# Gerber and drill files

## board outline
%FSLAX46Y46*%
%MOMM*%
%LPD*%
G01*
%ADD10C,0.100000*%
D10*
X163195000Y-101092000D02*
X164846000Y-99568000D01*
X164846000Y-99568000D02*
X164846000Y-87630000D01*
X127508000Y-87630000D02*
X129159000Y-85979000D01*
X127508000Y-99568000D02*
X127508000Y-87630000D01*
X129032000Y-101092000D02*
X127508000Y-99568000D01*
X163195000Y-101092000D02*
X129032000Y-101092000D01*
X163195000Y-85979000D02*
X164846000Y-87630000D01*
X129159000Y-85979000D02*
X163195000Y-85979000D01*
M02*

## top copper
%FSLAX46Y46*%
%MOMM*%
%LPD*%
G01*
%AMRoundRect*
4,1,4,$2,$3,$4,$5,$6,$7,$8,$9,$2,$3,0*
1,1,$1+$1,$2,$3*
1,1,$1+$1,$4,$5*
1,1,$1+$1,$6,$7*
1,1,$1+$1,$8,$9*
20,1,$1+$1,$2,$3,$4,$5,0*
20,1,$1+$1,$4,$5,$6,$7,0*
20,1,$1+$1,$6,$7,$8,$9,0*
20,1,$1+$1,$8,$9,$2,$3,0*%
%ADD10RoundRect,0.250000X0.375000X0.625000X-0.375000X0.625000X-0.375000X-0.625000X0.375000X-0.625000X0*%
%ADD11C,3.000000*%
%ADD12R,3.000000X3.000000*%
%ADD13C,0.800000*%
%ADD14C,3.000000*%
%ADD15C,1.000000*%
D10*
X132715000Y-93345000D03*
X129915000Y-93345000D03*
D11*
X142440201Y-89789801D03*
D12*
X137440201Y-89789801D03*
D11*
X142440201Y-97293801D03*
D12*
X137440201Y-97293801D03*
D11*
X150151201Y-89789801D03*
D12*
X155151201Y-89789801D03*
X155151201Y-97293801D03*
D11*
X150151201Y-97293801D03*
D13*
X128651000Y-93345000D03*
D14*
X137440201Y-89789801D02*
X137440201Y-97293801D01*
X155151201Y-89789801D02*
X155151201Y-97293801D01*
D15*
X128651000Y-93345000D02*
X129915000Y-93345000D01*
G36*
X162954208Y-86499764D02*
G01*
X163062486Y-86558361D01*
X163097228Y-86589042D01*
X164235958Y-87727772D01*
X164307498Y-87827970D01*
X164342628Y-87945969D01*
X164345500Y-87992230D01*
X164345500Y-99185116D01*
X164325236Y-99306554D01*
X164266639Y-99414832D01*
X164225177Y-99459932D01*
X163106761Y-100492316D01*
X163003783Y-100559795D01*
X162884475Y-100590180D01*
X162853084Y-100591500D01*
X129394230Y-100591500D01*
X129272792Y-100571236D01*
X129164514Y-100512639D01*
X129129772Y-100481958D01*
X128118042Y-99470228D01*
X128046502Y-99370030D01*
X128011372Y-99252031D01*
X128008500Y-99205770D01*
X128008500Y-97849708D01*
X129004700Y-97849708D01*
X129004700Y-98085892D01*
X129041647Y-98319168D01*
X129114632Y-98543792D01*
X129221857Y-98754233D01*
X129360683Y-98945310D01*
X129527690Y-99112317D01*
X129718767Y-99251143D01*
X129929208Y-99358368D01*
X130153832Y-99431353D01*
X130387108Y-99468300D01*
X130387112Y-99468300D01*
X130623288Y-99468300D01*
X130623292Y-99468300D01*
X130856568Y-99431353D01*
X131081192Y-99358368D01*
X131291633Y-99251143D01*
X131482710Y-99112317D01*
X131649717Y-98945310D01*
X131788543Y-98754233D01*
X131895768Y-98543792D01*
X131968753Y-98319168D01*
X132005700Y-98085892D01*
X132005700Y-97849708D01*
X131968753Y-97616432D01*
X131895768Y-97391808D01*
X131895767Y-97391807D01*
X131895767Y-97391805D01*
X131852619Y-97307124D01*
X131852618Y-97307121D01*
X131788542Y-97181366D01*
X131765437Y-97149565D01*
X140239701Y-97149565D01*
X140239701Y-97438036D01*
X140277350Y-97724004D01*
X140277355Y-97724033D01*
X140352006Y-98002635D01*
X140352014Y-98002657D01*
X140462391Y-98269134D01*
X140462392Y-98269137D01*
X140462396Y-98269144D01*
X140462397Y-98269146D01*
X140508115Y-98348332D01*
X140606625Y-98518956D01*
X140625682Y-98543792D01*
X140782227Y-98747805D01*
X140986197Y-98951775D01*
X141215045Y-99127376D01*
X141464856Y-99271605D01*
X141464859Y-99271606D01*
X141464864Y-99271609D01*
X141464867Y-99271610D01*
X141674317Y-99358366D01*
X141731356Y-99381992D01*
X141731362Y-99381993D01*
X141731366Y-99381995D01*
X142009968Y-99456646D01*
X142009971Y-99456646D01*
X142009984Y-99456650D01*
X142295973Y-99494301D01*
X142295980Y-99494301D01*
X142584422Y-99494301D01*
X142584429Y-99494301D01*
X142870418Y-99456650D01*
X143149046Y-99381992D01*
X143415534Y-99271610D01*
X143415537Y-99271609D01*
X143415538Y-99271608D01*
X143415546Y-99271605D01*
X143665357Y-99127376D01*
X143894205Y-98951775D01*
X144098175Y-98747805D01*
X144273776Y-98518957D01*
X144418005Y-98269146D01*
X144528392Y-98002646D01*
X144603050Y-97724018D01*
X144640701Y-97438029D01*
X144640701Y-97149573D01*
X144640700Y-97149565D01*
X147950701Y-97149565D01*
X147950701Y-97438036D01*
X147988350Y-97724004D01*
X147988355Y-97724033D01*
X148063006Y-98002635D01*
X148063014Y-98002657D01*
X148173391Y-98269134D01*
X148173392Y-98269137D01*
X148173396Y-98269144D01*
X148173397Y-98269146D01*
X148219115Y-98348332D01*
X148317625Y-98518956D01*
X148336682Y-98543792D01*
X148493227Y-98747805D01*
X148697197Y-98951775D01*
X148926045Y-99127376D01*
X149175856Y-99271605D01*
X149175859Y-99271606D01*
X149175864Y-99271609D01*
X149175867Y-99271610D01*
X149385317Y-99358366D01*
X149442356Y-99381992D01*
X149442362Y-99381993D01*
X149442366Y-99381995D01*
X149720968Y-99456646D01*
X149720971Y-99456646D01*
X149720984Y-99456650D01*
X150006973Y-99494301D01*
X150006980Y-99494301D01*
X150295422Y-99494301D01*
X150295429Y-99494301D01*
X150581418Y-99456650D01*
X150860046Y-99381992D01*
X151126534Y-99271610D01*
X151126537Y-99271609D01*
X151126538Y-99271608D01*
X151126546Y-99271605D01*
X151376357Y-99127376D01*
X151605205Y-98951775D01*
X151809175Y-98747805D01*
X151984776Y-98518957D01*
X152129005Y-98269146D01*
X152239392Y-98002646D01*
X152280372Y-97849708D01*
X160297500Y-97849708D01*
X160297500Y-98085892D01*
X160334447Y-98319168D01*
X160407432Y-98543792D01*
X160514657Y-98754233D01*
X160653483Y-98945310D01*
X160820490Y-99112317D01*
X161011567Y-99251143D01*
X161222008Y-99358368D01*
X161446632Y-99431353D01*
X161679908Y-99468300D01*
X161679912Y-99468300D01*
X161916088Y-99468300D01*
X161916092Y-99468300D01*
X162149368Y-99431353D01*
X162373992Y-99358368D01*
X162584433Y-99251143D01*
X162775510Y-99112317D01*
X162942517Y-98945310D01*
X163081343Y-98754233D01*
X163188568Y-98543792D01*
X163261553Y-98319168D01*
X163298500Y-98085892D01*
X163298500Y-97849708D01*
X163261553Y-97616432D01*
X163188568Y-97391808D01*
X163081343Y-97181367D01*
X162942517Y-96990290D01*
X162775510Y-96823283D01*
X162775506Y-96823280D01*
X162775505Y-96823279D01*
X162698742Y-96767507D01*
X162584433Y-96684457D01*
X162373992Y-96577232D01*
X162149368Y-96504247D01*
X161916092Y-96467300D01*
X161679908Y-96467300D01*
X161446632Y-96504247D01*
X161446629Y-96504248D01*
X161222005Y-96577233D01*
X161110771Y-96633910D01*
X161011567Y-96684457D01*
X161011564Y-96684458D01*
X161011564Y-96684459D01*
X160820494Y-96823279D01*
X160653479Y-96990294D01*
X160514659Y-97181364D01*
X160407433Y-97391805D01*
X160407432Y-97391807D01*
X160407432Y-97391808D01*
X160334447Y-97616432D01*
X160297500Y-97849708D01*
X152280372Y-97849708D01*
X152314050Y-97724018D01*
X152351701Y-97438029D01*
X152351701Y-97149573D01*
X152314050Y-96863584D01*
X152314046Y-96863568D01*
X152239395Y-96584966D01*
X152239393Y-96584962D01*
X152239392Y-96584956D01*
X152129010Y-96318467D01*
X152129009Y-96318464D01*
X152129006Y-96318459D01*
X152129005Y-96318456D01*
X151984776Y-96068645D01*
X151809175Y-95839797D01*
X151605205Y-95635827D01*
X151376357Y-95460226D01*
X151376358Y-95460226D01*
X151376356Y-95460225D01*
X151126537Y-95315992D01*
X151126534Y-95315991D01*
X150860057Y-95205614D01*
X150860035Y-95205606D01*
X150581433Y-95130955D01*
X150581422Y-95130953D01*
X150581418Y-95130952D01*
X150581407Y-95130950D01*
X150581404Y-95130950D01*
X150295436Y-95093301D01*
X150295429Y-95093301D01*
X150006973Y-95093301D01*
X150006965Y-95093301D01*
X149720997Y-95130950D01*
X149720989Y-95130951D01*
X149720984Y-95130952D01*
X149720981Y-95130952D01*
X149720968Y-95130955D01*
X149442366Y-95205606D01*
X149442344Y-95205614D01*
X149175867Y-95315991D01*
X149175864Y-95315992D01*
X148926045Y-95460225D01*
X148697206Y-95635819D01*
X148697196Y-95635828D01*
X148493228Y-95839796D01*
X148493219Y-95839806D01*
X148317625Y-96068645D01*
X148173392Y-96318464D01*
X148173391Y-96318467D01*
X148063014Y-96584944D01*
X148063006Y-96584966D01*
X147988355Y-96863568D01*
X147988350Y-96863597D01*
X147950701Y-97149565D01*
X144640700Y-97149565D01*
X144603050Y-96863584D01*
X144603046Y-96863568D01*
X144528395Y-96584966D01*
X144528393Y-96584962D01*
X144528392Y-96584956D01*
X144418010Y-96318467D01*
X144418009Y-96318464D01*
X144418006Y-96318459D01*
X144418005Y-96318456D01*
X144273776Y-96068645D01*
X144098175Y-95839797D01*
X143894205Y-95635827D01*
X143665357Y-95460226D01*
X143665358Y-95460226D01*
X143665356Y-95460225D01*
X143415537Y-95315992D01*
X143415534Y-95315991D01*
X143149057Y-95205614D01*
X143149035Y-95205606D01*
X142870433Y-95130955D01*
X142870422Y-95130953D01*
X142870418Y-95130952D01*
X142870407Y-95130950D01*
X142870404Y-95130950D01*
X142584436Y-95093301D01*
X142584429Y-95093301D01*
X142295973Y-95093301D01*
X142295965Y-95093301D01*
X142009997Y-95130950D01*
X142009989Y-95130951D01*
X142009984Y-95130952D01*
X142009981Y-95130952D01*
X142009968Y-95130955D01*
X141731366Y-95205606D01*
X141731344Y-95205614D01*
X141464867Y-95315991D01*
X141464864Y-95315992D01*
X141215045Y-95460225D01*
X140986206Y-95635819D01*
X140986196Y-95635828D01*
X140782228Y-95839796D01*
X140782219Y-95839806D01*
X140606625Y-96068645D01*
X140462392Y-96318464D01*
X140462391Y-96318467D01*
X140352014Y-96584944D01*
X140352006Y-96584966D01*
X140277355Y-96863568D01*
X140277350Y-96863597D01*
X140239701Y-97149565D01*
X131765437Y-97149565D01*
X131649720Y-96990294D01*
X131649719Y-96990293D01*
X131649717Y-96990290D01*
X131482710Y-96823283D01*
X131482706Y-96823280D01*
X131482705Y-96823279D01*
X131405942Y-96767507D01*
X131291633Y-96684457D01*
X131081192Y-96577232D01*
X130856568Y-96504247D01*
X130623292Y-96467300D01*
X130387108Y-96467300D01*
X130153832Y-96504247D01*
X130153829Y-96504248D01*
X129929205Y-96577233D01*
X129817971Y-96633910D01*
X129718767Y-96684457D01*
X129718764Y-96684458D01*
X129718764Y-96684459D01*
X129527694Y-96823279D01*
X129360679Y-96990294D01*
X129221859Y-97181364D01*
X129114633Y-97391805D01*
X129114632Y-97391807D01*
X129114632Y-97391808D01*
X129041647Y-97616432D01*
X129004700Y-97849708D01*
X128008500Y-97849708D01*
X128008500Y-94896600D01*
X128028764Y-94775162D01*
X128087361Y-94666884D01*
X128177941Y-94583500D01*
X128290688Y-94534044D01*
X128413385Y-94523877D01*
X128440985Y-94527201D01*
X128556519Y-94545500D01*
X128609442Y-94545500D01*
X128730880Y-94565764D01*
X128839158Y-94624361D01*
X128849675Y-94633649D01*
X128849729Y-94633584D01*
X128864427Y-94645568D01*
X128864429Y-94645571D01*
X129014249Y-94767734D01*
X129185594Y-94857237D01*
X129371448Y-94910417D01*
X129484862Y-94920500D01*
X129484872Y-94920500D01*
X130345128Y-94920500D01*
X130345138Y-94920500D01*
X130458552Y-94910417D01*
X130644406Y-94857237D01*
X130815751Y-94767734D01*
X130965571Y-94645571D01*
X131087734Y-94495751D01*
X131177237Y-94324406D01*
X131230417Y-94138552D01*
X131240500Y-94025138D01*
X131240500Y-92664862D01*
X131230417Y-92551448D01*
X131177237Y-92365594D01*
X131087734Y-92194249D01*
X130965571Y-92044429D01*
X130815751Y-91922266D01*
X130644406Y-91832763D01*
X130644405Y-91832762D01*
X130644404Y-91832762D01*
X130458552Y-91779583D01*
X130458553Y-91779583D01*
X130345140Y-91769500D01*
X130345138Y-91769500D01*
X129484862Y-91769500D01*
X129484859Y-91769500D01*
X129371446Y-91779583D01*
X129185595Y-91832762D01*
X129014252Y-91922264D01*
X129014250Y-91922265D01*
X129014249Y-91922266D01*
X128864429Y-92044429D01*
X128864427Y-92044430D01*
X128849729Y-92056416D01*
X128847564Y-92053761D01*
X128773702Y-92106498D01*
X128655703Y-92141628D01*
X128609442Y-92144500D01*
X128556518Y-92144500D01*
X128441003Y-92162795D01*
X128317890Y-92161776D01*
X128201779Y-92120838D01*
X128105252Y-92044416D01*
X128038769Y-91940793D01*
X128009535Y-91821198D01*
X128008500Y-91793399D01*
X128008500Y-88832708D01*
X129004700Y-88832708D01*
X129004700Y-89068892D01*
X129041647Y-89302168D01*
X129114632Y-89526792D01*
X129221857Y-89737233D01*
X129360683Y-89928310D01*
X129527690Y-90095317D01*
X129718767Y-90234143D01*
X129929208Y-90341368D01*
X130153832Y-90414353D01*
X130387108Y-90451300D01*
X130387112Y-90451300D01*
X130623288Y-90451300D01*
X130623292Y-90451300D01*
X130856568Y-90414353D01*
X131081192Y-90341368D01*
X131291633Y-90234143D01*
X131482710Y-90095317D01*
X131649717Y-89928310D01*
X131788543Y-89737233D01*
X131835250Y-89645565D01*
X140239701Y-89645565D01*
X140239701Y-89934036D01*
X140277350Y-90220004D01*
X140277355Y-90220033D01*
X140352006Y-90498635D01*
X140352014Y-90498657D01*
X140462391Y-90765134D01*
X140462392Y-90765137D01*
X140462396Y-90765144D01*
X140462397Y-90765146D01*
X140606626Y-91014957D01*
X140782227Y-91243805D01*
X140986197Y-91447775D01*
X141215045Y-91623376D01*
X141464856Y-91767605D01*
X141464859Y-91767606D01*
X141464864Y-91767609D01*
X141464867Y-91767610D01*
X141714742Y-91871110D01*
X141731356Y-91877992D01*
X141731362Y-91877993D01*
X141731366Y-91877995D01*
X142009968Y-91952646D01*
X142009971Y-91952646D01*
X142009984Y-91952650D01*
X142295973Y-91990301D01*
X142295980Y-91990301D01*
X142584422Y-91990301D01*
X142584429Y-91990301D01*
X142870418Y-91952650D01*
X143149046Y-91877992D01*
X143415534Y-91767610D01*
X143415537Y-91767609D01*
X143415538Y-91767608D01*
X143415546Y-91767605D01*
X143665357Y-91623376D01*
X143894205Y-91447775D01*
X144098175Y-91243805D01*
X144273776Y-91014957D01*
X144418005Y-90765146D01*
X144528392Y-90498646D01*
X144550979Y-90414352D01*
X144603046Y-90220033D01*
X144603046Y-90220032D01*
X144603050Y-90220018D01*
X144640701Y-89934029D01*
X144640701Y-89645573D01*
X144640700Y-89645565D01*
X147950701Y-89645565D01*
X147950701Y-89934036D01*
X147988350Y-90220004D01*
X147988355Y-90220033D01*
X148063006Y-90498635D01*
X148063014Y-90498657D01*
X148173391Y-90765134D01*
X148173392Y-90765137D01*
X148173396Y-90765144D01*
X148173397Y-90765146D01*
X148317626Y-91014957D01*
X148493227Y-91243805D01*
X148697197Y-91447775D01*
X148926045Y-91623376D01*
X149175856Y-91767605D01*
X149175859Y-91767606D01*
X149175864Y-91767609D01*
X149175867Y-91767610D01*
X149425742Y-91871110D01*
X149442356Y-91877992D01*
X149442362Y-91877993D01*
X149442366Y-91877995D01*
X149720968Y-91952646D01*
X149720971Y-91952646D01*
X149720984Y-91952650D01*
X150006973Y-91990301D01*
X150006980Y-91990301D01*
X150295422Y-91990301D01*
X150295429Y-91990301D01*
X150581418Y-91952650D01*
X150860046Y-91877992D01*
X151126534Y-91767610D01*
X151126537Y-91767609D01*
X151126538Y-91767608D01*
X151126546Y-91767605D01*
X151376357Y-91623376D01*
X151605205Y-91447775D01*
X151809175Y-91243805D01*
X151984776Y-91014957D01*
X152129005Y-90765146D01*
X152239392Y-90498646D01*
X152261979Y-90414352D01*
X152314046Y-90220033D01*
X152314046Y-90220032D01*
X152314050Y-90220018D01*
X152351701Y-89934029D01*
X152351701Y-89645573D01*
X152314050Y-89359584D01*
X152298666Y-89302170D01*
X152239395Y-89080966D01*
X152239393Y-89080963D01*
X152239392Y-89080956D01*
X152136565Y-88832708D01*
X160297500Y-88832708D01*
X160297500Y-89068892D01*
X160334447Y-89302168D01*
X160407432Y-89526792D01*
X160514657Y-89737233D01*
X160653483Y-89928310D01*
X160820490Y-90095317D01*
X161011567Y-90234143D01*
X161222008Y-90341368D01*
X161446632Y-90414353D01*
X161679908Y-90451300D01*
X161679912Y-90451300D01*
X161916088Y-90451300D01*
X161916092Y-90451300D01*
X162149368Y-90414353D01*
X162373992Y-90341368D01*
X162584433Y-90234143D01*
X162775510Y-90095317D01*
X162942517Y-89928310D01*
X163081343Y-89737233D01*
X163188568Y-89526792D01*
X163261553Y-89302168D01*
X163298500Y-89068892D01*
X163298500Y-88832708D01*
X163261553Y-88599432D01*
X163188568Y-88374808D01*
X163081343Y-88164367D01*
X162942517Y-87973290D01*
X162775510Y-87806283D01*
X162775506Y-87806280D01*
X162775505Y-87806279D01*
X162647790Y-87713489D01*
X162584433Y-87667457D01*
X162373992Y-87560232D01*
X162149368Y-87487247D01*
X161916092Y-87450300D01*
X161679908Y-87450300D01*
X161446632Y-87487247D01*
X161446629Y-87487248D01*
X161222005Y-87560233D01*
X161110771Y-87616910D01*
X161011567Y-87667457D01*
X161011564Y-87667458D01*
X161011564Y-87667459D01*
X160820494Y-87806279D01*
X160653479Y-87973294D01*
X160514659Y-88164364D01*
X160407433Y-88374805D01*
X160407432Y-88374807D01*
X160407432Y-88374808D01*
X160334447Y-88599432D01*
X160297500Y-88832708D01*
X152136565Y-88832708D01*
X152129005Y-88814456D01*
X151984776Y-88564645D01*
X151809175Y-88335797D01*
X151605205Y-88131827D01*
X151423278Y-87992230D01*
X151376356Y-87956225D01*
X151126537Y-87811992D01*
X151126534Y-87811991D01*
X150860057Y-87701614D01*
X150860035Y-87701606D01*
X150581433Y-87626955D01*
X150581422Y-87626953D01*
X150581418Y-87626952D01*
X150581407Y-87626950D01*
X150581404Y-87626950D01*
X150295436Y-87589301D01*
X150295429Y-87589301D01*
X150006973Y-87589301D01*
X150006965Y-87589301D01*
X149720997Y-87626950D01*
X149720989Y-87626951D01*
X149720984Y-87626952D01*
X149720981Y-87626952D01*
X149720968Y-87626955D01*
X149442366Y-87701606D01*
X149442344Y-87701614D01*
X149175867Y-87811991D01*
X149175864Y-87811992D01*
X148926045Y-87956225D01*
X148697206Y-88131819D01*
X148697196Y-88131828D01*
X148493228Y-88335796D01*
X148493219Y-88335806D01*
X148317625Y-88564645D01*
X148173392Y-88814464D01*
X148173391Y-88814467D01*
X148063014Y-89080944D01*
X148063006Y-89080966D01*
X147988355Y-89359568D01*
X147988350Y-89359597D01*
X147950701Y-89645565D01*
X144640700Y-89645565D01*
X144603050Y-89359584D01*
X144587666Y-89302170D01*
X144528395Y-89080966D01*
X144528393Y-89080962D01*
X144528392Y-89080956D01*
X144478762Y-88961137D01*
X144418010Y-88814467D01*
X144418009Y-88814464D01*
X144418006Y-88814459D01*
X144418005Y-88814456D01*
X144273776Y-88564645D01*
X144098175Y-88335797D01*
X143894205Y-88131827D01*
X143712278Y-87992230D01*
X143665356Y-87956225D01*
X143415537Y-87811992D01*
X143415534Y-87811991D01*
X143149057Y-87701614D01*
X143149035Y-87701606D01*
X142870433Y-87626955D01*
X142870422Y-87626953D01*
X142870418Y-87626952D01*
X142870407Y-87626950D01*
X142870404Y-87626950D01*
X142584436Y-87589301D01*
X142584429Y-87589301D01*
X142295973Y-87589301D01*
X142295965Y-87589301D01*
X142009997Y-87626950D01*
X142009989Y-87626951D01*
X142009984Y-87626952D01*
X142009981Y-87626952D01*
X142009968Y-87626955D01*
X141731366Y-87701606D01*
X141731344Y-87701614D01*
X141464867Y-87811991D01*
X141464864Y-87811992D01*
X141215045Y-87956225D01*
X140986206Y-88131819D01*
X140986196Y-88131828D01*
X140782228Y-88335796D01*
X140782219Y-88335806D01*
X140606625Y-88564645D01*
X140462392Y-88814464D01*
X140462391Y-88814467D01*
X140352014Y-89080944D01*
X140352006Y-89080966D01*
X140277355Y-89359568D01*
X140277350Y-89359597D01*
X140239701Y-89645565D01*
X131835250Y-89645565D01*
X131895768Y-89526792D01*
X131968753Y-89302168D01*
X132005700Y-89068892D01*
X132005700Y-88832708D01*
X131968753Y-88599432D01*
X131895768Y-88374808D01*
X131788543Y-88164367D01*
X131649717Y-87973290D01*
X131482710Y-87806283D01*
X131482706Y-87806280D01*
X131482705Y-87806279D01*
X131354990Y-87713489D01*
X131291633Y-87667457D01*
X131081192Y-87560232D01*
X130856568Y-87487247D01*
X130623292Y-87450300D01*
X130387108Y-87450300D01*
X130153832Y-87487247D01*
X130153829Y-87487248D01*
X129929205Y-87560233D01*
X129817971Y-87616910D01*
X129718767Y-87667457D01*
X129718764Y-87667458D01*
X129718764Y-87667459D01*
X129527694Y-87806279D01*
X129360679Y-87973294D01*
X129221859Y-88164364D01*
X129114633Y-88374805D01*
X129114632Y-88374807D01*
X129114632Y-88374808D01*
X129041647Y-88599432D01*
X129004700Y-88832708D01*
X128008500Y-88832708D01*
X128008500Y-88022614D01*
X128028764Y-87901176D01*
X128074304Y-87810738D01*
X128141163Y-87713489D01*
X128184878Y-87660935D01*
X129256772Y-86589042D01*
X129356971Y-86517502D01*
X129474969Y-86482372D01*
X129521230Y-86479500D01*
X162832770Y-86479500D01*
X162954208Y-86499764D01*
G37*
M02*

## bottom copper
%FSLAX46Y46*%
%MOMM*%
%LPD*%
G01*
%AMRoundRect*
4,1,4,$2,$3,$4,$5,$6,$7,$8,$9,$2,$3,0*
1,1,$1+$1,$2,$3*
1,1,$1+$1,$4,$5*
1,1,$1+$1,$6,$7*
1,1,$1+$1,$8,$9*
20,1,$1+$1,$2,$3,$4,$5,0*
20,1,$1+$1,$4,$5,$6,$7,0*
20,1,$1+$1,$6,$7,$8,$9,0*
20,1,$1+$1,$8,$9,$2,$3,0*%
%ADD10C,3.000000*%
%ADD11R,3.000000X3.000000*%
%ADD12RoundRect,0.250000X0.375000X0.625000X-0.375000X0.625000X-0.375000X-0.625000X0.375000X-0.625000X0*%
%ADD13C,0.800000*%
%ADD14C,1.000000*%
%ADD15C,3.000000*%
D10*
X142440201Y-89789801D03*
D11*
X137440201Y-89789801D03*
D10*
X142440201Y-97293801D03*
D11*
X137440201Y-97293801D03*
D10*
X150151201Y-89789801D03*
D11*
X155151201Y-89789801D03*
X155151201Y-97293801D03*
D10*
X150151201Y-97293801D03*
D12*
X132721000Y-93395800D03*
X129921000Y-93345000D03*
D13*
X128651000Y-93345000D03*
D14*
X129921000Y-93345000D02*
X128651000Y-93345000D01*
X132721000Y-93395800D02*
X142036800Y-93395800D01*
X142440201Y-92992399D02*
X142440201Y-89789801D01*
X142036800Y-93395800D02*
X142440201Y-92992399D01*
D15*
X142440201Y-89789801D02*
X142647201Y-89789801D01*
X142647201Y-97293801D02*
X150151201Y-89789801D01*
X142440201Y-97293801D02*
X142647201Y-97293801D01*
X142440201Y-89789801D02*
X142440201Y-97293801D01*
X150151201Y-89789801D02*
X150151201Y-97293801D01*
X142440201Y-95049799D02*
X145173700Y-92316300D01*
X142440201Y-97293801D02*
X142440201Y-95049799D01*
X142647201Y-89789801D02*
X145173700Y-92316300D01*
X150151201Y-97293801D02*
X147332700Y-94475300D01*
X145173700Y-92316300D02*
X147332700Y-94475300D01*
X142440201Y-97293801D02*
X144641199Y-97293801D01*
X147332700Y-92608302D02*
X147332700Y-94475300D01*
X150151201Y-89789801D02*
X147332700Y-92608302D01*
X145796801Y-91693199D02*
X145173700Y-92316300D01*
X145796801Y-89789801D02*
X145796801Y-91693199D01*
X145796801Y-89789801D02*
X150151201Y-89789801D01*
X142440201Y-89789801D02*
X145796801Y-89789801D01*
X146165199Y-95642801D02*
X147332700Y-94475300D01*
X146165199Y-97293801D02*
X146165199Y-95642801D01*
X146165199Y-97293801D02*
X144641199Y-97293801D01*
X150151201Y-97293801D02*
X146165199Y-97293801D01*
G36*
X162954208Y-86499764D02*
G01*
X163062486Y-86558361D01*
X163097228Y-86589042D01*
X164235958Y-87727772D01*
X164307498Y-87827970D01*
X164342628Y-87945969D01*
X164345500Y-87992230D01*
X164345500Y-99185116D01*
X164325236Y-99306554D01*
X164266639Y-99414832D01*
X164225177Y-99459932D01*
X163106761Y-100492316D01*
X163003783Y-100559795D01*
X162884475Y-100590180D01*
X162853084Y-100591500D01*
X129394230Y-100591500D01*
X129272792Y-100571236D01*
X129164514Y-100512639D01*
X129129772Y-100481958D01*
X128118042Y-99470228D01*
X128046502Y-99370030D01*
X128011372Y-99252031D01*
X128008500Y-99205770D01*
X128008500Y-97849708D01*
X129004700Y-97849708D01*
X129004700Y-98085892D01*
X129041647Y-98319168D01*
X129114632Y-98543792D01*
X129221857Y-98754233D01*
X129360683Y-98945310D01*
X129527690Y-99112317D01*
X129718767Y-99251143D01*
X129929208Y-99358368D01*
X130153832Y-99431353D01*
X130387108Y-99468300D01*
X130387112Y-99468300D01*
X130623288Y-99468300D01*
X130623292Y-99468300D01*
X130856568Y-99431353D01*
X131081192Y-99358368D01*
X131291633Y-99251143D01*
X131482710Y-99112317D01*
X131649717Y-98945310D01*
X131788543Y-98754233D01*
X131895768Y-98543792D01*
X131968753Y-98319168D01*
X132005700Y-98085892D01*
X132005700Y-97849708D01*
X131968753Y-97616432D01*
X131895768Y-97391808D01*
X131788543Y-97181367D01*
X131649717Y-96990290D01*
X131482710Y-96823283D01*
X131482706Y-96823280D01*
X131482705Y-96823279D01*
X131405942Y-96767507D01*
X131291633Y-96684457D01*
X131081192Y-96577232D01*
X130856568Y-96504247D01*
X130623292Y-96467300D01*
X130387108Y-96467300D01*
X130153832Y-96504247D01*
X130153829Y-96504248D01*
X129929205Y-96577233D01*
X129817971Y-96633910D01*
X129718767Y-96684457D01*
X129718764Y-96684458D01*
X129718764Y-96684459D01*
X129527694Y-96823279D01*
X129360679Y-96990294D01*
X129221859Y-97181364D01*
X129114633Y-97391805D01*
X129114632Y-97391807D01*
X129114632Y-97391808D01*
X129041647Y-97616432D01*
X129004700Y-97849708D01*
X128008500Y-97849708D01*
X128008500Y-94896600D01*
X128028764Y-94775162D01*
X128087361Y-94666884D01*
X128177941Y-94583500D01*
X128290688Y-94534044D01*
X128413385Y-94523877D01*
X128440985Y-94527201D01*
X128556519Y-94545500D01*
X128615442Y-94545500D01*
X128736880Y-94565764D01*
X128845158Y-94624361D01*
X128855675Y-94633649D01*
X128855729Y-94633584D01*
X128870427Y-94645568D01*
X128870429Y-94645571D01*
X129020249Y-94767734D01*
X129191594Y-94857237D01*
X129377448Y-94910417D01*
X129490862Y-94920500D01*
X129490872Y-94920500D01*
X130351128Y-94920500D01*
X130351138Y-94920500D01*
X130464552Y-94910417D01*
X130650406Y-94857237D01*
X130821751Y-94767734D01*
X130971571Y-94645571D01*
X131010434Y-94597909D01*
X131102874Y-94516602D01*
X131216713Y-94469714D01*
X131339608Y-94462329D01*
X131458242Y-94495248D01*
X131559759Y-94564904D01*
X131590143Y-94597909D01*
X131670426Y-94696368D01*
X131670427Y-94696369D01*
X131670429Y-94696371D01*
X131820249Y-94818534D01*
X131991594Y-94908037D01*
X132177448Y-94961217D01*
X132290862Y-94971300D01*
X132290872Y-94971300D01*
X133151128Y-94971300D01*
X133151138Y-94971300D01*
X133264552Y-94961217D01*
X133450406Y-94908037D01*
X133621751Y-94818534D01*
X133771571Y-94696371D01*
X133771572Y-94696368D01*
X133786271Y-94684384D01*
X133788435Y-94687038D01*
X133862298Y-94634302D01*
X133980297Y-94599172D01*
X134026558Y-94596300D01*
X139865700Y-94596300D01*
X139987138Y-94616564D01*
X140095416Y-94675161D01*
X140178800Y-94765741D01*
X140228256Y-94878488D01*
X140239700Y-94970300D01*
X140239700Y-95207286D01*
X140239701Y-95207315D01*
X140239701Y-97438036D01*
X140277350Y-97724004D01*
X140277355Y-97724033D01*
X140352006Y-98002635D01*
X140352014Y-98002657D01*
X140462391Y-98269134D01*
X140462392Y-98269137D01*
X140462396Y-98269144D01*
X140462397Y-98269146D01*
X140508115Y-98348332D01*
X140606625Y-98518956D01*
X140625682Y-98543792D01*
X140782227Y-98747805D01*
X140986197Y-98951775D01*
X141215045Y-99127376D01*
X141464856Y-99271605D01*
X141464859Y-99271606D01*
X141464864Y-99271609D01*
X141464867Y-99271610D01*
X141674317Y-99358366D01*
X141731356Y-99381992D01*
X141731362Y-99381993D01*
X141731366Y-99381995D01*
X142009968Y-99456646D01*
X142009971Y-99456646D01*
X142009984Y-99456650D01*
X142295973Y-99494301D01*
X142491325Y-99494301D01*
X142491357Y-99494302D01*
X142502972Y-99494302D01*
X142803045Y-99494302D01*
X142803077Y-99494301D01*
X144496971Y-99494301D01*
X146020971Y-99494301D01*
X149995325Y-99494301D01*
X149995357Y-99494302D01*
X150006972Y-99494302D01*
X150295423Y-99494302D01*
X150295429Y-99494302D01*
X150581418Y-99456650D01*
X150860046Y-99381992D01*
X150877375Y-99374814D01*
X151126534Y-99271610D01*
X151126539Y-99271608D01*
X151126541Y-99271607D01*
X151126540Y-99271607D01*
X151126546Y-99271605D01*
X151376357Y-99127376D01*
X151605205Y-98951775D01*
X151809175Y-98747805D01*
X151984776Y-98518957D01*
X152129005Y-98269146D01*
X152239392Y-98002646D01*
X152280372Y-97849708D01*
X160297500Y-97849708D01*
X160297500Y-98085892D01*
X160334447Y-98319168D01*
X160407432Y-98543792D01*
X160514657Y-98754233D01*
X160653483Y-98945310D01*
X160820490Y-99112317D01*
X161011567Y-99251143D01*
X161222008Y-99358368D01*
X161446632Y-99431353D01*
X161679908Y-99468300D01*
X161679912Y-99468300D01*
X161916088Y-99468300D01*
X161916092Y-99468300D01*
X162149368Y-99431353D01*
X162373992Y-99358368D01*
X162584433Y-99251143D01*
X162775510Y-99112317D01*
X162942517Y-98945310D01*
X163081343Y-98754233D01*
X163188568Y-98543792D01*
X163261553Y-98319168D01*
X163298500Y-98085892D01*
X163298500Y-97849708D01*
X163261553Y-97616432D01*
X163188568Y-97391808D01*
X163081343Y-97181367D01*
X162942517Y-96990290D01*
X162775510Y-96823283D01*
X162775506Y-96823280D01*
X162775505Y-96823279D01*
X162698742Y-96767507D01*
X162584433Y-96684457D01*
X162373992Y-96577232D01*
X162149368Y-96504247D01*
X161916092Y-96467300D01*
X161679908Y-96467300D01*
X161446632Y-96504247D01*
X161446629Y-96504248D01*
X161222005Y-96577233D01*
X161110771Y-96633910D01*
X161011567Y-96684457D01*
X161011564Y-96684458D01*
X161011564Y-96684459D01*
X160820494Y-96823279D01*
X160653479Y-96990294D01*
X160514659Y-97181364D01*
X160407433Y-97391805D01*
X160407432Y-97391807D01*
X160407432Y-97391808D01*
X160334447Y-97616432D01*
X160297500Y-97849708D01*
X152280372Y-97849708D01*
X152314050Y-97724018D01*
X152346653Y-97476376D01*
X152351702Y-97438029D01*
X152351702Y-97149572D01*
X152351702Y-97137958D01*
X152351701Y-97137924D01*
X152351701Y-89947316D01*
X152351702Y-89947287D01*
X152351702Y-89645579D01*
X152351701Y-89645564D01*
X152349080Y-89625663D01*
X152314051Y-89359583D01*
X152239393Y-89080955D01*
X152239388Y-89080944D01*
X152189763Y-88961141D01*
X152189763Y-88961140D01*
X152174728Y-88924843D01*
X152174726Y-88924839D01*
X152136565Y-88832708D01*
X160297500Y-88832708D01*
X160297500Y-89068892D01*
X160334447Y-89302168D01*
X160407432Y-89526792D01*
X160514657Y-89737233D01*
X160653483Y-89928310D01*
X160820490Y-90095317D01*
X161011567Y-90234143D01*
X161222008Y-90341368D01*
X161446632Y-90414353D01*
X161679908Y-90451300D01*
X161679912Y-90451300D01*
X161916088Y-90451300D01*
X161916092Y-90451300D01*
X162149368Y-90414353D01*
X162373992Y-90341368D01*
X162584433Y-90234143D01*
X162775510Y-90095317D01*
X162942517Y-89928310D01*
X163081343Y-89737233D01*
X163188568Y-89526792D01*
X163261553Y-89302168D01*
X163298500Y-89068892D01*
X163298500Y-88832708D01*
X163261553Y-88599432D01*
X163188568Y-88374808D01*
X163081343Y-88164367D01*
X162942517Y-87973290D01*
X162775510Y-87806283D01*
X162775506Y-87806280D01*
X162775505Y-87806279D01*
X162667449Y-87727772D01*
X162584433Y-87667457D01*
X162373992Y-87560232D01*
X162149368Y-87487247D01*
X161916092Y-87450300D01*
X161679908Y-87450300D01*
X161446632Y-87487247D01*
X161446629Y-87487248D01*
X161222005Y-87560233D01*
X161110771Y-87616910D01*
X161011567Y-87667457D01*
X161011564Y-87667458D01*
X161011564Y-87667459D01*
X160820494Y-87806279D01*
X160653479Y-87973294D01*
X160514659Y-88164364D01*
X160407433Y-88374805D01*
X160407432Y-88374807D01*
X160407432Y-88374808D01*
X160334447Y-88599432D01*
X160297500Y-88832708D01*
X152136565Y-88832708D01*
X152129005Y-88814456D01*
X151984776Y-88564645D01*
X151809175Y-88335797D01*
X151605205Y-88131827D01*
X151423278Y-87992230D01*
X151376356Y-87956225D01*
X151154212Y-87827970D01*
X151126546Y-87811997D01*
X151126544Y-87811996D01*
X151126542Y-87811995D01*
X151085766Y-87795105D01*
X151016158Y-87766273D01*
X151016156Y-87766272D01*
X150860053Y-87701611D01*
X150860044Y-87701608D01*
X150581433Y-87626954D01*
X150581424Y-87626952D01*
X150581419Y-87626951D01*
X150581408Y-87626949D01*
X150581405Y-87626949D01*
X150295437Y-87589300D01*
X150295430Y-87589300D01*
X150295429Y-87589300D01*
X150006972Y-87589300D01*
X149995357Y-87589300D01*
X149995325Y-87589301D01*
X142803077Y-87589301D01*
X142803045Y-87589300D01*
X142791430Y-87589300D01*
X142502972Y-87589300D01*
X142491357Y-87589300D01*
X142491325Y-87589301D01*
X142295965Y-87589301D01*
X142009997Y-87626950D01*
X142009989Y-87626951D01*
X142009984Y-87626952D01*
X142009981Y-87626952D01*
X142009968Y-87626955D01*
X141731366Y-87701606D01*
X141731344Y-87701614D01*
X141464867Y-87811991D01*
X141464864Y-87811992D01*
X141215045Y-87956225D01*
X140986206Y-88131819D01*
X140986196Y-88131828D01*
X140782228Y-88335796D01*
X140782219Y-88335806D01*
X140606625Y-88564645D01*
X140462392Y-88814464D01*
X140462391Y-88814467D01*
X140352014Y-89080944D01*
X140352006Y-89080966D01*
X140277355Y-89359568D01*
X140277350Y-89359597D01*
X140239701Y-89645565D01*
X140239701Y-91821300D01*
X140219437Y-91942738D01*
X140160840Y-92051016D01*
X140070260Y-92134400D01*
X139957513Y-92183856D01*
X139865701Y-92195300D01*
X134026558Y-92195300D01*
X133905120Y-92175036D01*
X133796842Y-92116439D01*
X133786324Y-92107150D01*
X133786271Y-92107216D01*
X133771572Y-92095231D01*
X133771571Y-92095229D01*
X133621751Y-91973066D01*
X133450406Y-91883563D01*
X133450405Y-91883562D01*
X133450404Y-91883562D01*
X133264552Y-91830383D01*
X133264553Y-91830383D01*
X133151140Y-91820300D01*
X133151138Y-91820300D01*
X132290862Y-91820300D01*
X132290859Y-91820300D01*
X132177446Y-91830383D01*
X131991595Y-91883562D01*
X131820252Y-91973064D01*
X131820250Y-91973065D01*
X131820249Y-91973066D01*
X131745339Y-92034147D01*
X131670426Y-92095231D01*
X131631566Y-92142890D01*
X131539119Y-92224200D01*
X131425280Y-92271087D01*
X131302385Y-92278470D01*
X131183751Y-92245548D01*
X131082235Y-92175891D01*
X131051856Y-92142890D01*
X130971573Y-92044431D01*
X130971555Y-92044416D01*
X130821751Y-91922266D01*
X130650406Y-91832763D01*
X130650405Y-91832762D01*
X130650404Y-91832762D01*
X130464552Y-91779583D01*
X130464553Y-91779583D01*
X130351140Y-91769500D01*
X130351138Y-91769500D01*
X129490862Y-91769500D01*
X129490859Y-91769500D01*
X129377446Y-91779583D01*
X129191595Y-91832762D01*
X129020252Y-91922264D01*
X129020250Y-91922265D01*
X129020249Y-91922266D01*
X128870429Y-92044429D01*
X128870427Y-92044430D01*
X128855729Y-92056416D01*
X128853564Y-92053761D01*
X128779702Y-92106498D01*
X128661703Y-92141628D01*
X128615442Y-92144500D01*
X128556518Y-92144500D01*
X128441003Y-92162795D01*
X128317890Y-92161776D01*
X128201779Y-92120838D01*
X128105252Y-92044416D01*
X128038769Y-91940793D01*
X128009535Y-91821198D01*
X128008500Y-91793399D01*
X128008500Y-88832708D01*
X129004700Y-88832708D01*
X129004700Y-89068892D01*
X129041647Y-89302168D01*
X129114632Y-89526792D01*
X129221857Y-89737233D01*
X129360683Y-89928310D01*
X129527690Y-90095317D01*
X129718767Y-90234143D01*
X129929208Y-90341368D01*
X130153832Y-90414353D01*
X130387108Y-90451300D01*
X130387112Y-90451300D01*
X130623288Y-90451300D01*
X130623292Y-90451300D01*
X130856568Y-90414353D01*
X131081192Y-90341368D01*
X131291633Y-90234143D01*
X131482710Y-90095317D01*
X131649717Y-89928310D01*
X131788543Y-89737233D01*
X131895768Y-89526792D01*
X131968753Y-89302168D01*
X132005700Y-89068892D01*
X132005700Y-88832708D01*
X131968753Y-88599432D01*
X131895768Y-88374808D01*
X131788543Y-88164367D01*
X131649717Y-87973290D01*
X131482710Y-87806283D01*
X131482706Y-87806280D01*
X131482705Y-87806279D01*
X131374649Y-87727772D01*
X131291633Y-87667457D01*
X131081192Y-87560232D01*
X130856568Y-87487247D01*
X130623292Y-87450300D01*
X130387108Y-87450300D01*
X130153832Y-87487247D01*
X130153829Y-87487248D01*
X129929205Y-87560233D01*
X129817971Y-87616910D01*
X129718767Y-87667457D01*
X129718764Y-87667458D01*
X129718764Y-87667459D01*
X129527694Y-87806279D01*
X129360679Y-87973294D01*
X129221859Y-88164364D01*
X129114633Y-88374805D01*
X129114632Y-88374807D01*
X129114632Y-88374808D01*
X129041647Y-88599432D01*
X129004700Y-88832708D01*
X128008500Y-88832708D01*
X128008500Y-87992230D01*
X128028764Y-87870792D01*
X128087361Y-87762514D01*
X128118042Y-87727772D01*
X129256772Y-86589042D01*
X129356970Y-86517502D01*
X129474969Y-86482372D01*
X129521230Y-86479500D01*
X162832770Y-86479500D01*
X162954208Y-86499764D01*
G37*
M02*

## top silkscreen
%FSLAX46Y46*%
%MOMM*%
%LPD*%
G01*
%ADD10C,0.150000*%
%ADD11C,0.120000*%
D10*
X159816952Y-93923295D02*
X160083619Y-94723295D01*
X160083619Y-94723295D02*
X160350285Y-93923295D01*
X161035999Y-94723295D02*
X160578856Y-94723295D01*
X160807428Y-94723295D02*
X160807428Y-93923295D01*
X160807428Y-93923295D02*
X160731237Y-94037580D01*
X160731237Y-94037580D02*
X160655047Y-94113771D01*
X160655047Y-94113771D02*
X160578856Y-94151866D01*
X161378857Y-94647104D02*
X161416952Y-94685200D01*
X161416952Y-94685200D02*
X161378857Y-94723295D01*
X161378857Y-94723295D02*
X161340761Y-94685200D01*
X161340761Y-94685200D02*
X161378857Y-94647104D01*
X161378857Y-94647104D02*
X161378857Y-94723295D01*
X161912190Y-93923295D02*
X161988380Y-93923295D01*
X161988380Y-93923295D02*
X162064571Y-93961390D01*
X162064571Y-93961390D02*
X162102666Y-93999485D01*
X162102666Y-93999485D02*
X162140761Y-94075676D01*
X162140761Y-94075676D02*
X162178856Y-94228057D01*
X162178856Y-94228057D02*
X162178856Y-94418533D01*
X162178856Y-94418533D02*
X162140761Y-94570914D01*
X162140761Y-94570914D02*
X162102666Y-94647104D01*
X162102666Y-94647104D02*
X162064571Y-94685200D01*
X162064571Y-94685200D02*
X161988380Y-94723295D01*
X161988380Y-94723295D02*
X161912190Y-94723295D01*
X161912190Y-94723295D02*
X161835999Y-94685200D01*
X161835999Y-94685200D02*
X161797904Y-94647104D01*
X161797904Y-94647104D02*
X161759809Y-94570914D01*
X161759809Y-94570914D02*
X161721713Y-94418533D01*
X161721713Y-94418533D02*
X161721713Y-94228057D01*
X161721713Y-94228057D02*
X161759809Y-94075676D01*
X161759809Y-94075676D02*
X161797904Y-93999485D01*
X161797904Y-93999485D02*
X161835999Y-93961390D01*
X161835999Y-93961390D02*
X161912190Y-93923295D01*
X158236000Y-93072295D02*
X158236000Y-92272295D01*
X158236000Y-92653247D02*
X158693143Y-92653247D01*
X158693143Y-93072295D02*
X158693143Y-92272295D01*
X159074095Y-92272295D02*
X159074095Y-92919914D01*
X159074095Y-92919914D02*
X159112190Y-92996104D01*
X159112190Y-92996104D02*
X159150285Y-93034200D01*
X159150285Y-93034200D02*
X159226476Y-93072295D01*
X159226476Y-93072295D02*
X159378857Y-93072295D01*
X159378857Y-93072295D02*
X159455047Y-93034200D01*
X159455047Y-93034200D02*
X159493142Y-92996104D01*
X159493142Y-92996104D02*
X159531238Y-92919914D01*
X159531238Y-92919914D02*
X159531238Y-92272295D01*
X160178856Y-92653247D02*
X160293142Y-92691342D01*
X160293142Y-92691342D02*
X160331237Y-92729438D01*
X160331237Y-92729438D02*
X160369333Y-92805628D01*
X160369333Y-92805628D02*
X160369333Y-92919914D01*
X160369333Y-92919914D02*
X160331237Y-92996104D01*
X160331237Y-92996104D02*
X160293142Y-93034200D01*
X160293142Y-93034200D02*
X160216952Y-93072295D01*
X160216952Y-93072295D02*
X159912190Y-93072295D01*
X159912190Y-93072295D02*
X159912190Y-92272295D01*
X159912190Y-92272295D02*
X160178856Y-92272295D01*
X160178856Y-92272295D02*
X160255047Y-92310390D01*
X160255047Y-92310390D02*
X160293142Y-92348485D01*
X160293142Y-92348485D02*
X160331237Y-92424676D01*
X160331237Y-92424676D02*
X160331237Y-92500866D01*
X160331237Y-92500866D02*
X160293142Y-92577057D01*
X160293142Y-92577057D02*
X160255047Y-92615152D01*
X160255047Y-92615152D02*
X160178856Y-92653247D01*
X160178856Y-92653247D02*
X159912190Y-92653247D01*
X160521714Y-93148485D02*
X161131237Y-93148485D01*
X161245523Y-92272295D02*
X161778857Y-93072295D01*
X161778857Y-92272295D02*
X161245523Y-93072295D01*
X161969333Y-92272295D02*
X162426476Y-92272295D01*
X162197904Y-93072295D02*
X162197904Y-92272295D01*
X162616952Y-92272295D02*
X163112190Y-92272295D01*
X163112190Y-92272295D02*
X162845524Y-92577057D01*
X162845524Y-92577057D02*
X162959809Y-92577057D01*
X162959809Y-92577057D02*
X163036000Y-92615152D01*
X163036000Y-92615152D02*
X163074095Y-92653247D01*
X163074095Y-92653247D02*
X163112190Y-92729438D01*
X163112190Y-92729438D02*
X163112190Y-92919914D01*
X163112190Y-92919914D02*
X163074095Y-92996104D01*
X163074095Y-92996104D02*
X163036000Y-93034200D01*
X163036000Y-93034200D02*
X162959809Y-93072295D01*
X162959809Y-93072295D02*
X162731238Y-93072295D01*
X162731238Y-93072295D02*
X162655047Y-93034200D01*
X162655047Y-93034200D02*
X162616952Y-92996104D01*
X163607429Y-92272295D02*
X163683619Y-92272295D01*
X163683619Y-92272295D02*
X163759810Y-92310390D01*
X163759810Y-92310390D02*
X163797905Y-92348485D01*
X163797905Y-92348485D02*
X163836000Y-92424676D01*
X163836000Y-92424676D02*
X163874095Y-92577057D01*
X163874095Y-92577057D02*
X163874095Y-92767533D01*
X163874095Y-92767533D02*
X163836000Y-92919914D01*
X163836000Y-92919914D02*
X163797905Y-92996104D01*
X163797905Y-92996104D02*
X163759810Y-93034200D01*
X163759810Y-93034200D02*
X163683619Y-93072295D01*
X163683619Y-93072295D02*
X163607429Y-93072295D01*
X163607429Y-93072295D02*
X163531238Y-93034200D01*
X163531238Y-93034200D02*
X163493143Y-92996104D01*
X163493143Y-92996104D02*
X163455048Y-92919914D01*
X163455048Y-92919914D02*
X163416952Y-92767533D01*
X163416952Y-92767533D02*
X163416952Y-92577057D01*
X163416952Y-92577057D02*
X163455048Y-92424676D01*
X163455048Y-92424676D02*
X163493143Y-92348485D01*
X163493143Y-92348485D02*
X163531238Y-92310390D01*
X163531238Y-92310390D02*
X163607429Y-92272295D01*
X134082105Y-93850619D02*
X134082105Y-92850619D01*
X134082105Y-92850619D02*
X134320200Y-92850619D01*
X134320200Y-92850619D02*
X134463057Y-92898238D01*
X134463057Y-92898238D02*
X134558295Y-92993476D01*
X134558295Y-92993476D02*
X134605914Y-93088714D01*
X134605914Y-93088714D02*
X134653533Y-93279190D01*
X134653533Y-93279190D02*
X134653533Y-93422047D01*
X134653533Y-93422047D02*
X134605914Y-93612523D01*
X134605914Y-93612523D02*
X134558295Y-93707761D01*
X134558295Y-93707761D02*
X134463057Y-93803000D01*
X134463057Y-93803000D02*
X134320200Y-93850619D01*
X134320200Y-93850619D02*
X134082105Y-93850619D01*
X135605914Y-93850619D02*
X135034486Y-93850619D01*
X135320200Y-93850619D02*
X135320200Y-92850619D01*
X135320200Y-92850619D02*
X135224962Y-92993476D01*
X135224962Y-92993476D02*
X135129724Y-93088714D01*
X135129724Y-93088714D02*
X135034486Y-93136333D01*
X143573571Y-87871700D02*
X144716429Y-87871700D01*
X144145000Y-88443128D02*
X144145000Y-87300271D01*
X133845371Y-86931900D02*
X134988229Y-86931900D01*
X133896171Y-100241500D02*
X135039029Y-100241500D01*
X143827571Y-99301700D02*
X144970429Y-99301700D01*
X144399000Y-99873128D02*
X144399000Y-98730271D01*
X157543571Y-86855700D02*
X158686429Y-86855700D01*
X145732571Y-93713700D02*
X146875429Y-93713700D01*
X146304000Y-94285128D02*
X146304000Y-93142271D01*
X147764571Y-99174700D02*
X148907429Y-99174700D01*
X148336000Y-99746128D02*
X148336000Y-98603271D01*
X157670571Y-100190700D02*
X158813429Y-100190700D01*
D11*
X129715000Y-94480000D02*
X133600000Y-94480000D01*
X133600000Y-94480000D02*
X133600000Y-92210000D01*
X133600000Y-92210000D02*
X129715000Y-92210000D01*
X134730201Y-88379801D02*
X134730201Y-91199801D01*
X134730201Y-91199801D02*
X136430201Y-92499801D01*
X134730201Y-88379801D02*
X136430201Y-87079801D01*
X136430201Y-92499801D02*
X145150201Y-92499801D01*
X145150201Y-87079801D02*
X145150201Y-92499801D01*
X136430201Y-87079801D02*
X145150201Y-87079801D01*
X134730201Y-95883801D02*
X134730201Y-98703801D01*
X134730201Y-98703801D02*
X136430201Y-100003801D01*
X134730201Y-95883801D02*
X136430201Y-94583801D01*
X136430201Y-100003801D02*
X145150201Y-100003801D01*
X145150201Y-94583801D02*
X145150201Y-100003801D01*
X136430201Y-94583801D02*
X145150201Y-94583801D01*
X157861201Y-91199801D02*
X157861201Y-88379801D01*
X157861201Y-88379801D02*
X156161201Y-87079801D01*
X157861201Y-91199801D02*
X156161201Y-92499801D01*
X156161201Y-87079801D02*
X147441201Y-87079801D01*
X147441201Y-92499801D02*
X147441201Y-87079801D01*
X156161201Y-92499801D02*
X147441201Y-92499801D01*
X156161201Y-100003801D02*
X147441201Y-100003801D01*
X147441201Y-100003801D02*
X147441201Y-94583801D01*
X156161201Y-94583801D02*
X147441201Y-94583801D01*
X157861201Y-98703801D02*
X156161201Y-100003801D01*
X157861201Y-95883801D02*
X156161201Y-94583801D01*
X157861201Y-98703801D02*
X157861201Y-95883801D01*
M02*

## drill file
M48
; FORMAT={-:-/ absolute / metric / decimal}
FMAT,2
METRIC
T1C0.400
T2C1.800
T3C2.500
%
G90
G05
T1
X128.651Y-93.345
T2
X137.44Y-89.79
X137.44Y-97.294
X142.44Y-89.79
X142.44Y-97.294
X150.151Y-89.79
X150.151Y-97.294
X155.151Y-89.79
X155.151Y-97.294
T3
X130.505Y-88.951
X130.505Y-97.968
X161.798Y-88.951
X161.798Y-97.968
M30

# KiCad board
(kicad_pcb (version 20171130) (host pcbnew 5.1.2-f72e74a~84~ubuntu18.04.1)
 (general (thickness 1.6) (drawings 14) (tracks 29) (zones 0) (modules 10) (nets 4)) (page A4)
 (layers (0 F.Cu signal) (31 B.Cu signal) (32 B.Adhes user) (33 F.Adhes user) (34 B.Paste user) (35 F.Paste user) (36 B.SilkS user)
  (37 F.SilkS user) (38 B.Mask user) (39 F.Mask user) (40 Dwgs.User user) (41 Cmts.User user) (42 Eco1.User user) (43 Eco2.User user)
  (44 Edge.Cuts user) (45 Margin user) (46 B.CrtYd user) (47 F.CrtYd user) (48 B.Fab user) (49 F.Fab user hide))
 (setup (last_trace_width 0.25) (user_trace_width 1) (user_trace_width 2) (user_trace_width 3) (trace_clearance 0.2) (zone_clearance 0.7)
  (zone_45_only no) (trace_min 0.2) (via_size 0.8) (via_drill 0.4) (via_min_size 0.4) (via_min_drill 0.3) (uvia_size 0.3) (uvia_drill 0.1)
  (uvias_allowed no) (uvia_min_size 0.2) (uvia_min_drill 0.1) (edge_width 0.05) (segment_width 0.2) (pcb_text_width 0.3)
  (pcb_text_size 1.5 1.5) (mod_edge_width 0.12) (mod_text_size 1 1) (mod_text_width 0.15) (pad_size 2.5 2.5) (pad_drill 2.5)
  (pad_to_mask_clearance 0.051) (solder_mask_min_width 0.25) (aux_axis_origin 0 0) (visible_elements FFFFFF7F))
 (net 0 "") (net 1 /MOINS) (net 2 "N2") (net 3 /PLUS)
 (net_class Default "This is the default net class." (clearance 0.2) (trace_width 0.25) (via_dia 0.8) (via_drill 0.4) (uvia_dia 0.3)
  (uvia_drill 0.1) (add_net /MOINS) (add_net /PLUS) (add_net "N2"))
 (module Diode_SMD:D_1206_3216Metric (layer F.Cu) (at 131.315 93.345 180)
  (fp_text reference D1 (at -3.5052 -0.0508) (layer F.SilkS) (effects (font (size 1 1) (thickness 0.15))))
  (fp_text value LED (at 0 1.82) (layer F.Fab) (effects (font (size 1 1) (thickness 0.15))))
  (fp_line (start 1.6 -1.135) (end -2.285 -1.135) (layer F.SilkS) (width 0.12))
  (fp_line (start -2.285 -1.135) (end -2.285 1.135) (layer F.SilkS) (width 0.12))
  (fp_line (start -2.285 1.135) (end 1.6 1.135) (layer F.SilkS) (width 0.12))
  (pad 1 smd roundrect (at -1.4 0 180) (size 1.25 1.75) (layers F.Cu F.Paste F.Mask) (roundrect_rratio 0.2) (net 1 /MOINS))
  (pad 2 smd roundrect (at 1.4 0 180) (size 1.25 1.75) (layers F.Cu F.Paste F.Mask) (roundrect_rratio 0.2) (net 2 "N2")))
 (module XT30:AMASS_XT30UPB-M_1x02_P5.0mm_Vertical (layer F.Cu) (at 137.440201 89.789801)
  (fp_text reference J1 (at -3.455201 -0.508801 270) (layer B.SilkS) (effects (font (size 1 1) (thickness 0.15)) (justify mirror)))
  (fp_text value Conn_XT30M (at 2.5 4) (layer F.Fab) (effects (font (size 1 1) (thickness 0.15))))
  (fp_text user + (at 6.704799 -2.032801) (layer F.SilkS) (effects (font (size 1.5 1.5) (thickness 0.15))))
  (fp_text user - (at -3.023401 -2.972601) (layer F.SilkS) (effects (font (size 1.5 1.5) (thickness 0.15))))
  (fp_line (start -2.71 -1.41) (end -2.71 1.41) (layer F.SilkS) (width 0.12))
  (fp_line (start -2.71 1.41) (end -1.01 2.71) (layer F.SilkS) (width 0.12))
  (fp_line (start -2.71 -1.41) (end -1.01 -2.71) (layer F.SilkS) (width 0.12))
  (fp_line (start -1.01 2.71) (end 7.71 2.71) (layer F.SilkS) (width 0.12))
  (fp_line (start 7.71 -2.71) (end 7.71 2.71) (layer F.SilkS) (width 0.12))
  (fp_line (start -1.01 -2.71) (end 7.71 -2.71) (layer F.SilkS) (width 0.12))
  (pad 2 thru_hole circle (at 5 0) (size 3 3) (drill 1.8) (layers *.Cu *.Mask) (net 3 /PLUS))
  (pad 1 thru_hole rect (at 0 0) (size 3 3) (drill 1.8) (layers *.Cu *.Mask) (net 1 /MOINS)))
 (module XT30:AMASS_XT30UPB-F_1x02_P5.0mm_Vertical (layer F.Cu) (at 137.440201 97.293801)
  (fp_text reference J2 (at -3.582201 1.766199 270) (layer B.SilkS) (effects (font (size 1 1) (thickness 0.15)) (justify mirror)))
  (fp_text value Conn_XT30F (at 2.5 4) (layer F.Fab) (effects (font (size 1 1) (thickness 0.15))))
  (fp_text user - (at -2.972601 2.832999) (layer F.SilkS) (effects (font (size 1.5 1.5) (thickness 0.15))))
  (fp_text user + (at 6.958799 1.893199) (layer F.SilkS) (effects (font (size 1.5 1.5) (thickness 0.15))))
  (fp_line (start -2.71 -1.41) (end -2.71 1.41) (layer F.SilkS) (width 0.12))
  (fp_line (start -2.71 1.41) (end -1.01 2.71) (layer F.SilkS) (width 0.12))
  (fp_line (start -2.71 -1.41) (end -1.01 -2.71) (layer F.SilkS) (width 0.12))
  (fp_line (start -1.01 2.71) (end 7.71 2.71) (layer F.SilkS) (width 0.12))
  (fp_line (start 7.71 -2.71) (end 7.71 2.71) (layer F.SilkS) (width 0.12))
  (fp_line (start -1.01 -2.71) (end 7.71 -2.71) (layer F.SilkS) (width 0.12))
  (pad 2 thru_hole circle (at 5 0) (size 3 3) (drill 1.8) (layers *.Cu *.Mask) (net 3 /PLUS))
  (pad 1 thru_hole rect (at 0 0) (size 3 3) (drill 1.8) (layers *.Cu *.Mask) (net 1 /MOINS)))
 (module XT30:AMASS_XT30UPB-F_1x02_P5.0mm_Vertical (layer F.Cu) (at 155.151201 89.789801 180)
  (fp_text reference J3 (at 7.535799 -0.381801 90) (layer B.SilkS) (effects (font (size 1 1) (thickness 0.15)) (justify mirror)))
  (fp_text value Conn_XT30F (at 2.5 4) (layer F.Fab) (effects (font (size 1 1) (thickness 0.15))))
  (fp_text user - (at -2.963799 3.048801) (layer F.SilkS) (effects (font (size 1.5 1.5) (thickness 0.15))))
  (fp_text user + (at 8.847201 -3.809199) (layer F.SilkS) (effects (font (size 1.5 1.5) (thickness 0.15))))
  (fp_line (start -2.71 -1.41) (end -2.71 1.41) (layer F.SilkS) (width 0.12))
  (fp_line (start -2.71 1.41) (end -1.01 2.71) (layer F.SilkS) (width 0.12))
  (fp_line (start -2.71 -1.41) (end -1.01 -2.71) (layer F.SilkS) (width 0.12))
  (fp_line (start -1.01 2.71) (end 7.71 2.71) (layer F.SilkS) (width 0.12))
  (fp_line (start 7.71 -2.71) (end 7.71 2.71) (layer F.SilkS) (width 0.12))
  (fp_line (start -1.01 -2.71) (end 7.71 -2.71) (layer F.SilkS) (width 0.12))
  (pad 2 thru_hole circle (at 5 0 180) (size 3 3) (drill 1.8) (layers *.Cu *.Mask) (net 3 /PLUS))
  (pad 1 thru_hole rect (at 0 0 180) (size 3 3) (drill 1.8) (layers *.Cu *.Mask) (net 1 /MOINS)))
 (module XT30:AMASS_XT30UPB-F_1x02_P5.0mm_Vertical (layer F.Cu) (at 155.151201 97.293801 180)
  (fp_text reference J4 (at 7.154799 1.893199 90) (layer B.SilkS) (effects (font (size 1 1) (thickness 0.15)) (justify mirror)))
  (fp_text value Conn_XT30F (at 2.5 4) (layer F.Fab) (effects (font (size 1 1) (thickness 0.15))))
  (fp_line (start -1.01 -2.71) (end 7.71 -2.71) (layer F.SilkS) (width 0.12))
  (fp_line (start 7.71 -2.71) (end 7.71 2.71) (layer F.SilkS) (width 0.12))
  (fp_line (start -1.01 2.71) (end 7.71 2.71) (layer F.SilkS) (width 0.12))
  (fp_line (start -2.71 -1.41) (end -1.01 -2.71) (layer F.SilkS) (width 0.12))
  (fp_line (start -2.71 1.41) (end -1.01 2.71) (layer F.SilkS) (width 0.12))
  (fp_line (start -2.71 -1.41) (end -2.71 1.41) (layer F.SilkS) (width 0.12))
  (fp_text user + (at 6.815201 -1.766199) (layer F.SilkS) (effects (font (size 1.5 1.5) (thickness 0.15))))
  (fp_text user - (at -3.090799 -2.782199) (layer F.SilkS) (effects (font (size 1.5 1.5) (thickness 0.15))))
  (pad 1 thru_hole rect (at 0 0 180) (size 3 3) (drill 1.8) (layers *.Cu *.Mask) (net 1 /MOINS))
  (pad 2 thru_hole circle (at 5 0 180) (size 3 3) (drill 1.8) (layers *.Cu *.Mask) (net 3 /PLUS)))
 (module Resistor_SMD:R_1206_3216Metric (layer B.Cu) (at 131.321 93.3958 180)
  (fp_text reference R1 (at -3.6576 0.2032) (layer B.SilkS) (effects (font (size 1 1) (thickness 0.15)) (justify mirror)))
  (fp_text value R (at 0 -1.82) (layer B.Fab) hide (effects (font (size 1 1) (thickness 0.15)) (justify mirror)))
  (pad 1 smd roundrect (at -1.4 0 180) (size 1.25 1.75) (layers B.Cu B.Paste B.Mask) (roundrect_rratio 0.2) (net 3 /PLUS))
  (pad 2 smd roundrect (at 1.4 0.0508 180) (size 1.25 1.75) (layers B.Cu B.Paste B.Mask) (roundrect_rratio 0.2) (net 2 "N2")))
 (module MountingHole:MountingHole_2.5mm (layer F.Cu) (at 130.5052 88.9508)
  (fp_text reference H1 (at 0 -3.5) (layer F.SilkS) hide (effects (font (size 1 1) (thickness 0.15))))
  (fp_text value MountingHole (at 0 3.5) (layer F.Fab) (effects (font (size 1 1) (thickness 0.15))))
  (pad "" np_thru_hole circle (at 0 0) (size 2.5 2.5) (drill 2.5) (layers *.Cu *.Mask)))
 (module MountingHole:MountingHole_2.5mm (layer F.Cu) (at 161.798 88.9508)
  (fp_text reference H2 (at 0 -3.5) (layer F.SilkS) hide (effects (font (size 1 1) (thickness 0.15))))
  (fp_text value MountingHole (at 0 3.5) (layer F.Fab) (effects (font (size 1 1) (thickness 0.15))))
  (pad "" np_thru_hole circle (at 0 0) (size 2.5 2.5) (drill 2.5) (layers *.Cu *.Mask)))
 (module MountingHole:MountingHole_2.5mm (layer F.Cu) (at 130.5052 97.9678)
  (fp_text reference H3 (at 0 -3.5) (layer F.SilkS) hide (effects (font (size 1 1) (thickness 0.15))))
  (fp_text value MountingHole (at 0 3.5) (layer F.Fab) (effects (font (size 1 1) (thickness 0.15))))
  (pad 1 np_thru_hole circle (at 0 0) (size 2.5 2.5) (drill 2.5) (layers *.Cu *.Mask)))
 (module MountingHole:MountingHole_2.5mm (layer F.Cu) (at 161.798 97.9678)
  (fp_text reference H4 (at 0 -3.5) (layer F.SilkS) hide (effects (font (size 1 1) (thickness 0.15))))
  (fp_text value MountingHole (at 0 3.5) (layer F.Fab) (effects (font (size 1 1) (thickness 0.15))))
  (pad 1 np_thru_hole circle (at 0 0) (size 2.5 2.5) (drill 2.5) (layers *.Cu *.Mask)))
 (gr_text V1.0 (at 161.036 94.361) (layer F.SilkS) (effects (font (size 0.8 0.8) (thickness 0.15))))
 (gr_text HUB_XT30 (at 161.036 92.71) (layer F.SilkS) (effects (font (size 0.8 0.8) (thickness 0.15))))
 (gr_line (start 163.195 101.092) (end 164.846 99.568) (layer Edge.Cuts) (width 0.1))
 (gr_line (start 164.846 99.568) (end 164.846 87.63) (layer Edge.Cuts) (width 0.1))
 (gr_line (start 127.508 87.63) (end 129.159 85.979) (layer Edge.Cuts) (width 0.1))
 (gr_line (start 127.508 99.568) (end 127.508 87.63) (layer Edge.Cuts) (width 0.1))
 (gr_line (start 129.032 101.092) (end 127.508 99.568) (layer Edge.Cuts) (width 0.1))
 (gr_line (start 163.195 101.092) (end 129.032 101.092) (layer Edge.Cuts) (width 0.1))
 (gr_line (start 163.195 85.979) (end 164.846 87.63) (layer Edge.Cuts) (width 0.1))
 (gr_line (start 129.159 85.979) (end 163.195 85.979) (layer Edge.Cuts) (width 0.1))
 (segment (start 137.440201 89.789801) (end 137.440201 97.293801) (width 3) (layer F.Cu) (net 1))
 (segment (start 155.151201 89.789801) (end 155.151201 97.293801) (width 3) (layer F.Cu) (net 1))
 (via (at 128.651 93.345) (size 0.8) (drill 0.4) (layers F.Cu B.Cu) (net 2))
 (segment (start 129.921 93.345) (end 128.651 93.345) (width 1) (layer B.Cu) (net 2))
 (segment (start 128.651 93.345) (end 129.915 93.345) (width 1) (layer F.Cu) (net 2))
 (segment (start 132.721 93.3958) (end 142.0368 93.3958) (width 1) (layer B.Cu) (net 3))
 (segment (start 142.440201 92.992399) (end 142.440201 89.789801) (width 1) (layer B.Cu) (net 3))
 (segment (start 142.0368 93.3958) (end 142.440201 92.992399) (width 1) (layer B.Cu) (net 3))
 (segment (start 142.440201 89.789801) (end 142.647201 89.789801) (width 3) (layer B.Cu) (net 3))
 (segment (start 142.647201 97.293801) (end 150.151201 89.789801) (width 3) (layer B.Cu) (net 3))
 (segment (start 142.440201 97.293801) (end 142.647201 97.293801) (width 3) (layer B.Cu) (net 3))
 (segment (start 142.440201 89.789801) (end 142.440201 97.293801) (width 3) (layer B.Cu) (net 3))
 (segment (start 150.151201 89.789801) (end 150.151201 97.293801) (width 3) (layer B.Cu) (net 3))
 (segment (start 142.440201 95.049799) (end 145.1737 92.3163) (width 3) (layer B.Cu) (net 3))
 (segment (start 142.440201 97.293801) (end 142.440201 95.049799) (width 3) (layer B.Cu) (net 3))
 (segment (start 142.647201 89.789801) (end 145.1737 92.3163) (width 3) (layer B.Cu) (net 3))
 (segment (start 150.151201 97.293801) (end 147.3327 94.4753) (width 3) (layer B.Cu) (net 3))
 (segment (start 145.1737 92.3163) (end 147.3327 94.4753) (width 3) (layer B.Cu) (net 3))
 (segment (start 142.440201 97.293801) (end 144.641199 97.293801) (width 3) (layer B.Cu) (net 3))
 (segment (start 147.3327 92.608302) (end 147.3327 94.4753) (width 3) (layer B.Cu) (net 3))
 (segment (start 150.151201 89.789801) (end 147.3327 92.608302) (width 3) (layer B.Cu) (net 3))
 (segment (start 145.796801 91.693199) (end 145.1737 92.3163) (width 3) (layer B.Cu) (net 3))
 (segment (start 145.796801 89.789801) (end 145.796801 91.693199) (width 3) (layer B.Cu) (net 3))
 (segment (start 145.796801 89.789801) (end 150.151201 89.789801) (width 3) (layer B.Cu) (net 3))
 (segment (start 142.440201 89.789801) (end 145.796801 89.789801) (width 3) (layer B.Cu) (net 3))
 (segment (start 146.165199 95.642801) (end 147.3327 94.4753) (width 3) (layer B.Cu) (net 3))
 (segment (start 146.165199 97.293801) (end 146.165199 95.642801) (width 3) (layer B.Cu) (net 3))
 (segment (start 146.165199 97.293801) (end 144.641199 97.293801) (width 3) (layer B.Cu) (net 3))
 (segment (start 150.151201 97.293801) (end 146.165199 97.293801) (width 3) (layer B.Cu) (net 3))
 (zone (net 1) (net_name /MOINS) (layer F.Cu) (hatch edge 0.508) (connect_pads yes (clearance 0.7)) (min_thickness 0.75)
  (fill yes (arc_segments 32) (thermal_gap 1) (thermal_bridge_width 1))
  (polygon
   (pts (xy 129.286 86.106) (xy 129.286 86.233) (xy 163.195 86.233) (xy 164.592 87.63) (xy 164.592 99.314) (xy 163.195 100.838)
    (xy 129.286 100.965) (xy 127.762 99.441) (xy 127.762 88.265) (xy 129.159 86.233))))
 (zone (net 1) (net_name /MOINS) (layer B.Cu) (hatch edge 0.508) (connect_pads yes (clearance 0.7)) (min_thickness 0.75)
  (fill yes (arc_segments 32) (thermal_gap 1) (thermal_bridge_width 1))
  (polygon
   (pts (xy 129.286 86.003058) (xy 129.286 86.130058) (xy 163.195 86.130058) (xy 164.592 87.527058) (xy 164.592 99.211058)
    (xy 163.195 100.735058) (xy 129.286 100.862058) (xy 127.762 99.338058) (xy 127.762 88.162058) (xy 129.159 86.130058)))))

